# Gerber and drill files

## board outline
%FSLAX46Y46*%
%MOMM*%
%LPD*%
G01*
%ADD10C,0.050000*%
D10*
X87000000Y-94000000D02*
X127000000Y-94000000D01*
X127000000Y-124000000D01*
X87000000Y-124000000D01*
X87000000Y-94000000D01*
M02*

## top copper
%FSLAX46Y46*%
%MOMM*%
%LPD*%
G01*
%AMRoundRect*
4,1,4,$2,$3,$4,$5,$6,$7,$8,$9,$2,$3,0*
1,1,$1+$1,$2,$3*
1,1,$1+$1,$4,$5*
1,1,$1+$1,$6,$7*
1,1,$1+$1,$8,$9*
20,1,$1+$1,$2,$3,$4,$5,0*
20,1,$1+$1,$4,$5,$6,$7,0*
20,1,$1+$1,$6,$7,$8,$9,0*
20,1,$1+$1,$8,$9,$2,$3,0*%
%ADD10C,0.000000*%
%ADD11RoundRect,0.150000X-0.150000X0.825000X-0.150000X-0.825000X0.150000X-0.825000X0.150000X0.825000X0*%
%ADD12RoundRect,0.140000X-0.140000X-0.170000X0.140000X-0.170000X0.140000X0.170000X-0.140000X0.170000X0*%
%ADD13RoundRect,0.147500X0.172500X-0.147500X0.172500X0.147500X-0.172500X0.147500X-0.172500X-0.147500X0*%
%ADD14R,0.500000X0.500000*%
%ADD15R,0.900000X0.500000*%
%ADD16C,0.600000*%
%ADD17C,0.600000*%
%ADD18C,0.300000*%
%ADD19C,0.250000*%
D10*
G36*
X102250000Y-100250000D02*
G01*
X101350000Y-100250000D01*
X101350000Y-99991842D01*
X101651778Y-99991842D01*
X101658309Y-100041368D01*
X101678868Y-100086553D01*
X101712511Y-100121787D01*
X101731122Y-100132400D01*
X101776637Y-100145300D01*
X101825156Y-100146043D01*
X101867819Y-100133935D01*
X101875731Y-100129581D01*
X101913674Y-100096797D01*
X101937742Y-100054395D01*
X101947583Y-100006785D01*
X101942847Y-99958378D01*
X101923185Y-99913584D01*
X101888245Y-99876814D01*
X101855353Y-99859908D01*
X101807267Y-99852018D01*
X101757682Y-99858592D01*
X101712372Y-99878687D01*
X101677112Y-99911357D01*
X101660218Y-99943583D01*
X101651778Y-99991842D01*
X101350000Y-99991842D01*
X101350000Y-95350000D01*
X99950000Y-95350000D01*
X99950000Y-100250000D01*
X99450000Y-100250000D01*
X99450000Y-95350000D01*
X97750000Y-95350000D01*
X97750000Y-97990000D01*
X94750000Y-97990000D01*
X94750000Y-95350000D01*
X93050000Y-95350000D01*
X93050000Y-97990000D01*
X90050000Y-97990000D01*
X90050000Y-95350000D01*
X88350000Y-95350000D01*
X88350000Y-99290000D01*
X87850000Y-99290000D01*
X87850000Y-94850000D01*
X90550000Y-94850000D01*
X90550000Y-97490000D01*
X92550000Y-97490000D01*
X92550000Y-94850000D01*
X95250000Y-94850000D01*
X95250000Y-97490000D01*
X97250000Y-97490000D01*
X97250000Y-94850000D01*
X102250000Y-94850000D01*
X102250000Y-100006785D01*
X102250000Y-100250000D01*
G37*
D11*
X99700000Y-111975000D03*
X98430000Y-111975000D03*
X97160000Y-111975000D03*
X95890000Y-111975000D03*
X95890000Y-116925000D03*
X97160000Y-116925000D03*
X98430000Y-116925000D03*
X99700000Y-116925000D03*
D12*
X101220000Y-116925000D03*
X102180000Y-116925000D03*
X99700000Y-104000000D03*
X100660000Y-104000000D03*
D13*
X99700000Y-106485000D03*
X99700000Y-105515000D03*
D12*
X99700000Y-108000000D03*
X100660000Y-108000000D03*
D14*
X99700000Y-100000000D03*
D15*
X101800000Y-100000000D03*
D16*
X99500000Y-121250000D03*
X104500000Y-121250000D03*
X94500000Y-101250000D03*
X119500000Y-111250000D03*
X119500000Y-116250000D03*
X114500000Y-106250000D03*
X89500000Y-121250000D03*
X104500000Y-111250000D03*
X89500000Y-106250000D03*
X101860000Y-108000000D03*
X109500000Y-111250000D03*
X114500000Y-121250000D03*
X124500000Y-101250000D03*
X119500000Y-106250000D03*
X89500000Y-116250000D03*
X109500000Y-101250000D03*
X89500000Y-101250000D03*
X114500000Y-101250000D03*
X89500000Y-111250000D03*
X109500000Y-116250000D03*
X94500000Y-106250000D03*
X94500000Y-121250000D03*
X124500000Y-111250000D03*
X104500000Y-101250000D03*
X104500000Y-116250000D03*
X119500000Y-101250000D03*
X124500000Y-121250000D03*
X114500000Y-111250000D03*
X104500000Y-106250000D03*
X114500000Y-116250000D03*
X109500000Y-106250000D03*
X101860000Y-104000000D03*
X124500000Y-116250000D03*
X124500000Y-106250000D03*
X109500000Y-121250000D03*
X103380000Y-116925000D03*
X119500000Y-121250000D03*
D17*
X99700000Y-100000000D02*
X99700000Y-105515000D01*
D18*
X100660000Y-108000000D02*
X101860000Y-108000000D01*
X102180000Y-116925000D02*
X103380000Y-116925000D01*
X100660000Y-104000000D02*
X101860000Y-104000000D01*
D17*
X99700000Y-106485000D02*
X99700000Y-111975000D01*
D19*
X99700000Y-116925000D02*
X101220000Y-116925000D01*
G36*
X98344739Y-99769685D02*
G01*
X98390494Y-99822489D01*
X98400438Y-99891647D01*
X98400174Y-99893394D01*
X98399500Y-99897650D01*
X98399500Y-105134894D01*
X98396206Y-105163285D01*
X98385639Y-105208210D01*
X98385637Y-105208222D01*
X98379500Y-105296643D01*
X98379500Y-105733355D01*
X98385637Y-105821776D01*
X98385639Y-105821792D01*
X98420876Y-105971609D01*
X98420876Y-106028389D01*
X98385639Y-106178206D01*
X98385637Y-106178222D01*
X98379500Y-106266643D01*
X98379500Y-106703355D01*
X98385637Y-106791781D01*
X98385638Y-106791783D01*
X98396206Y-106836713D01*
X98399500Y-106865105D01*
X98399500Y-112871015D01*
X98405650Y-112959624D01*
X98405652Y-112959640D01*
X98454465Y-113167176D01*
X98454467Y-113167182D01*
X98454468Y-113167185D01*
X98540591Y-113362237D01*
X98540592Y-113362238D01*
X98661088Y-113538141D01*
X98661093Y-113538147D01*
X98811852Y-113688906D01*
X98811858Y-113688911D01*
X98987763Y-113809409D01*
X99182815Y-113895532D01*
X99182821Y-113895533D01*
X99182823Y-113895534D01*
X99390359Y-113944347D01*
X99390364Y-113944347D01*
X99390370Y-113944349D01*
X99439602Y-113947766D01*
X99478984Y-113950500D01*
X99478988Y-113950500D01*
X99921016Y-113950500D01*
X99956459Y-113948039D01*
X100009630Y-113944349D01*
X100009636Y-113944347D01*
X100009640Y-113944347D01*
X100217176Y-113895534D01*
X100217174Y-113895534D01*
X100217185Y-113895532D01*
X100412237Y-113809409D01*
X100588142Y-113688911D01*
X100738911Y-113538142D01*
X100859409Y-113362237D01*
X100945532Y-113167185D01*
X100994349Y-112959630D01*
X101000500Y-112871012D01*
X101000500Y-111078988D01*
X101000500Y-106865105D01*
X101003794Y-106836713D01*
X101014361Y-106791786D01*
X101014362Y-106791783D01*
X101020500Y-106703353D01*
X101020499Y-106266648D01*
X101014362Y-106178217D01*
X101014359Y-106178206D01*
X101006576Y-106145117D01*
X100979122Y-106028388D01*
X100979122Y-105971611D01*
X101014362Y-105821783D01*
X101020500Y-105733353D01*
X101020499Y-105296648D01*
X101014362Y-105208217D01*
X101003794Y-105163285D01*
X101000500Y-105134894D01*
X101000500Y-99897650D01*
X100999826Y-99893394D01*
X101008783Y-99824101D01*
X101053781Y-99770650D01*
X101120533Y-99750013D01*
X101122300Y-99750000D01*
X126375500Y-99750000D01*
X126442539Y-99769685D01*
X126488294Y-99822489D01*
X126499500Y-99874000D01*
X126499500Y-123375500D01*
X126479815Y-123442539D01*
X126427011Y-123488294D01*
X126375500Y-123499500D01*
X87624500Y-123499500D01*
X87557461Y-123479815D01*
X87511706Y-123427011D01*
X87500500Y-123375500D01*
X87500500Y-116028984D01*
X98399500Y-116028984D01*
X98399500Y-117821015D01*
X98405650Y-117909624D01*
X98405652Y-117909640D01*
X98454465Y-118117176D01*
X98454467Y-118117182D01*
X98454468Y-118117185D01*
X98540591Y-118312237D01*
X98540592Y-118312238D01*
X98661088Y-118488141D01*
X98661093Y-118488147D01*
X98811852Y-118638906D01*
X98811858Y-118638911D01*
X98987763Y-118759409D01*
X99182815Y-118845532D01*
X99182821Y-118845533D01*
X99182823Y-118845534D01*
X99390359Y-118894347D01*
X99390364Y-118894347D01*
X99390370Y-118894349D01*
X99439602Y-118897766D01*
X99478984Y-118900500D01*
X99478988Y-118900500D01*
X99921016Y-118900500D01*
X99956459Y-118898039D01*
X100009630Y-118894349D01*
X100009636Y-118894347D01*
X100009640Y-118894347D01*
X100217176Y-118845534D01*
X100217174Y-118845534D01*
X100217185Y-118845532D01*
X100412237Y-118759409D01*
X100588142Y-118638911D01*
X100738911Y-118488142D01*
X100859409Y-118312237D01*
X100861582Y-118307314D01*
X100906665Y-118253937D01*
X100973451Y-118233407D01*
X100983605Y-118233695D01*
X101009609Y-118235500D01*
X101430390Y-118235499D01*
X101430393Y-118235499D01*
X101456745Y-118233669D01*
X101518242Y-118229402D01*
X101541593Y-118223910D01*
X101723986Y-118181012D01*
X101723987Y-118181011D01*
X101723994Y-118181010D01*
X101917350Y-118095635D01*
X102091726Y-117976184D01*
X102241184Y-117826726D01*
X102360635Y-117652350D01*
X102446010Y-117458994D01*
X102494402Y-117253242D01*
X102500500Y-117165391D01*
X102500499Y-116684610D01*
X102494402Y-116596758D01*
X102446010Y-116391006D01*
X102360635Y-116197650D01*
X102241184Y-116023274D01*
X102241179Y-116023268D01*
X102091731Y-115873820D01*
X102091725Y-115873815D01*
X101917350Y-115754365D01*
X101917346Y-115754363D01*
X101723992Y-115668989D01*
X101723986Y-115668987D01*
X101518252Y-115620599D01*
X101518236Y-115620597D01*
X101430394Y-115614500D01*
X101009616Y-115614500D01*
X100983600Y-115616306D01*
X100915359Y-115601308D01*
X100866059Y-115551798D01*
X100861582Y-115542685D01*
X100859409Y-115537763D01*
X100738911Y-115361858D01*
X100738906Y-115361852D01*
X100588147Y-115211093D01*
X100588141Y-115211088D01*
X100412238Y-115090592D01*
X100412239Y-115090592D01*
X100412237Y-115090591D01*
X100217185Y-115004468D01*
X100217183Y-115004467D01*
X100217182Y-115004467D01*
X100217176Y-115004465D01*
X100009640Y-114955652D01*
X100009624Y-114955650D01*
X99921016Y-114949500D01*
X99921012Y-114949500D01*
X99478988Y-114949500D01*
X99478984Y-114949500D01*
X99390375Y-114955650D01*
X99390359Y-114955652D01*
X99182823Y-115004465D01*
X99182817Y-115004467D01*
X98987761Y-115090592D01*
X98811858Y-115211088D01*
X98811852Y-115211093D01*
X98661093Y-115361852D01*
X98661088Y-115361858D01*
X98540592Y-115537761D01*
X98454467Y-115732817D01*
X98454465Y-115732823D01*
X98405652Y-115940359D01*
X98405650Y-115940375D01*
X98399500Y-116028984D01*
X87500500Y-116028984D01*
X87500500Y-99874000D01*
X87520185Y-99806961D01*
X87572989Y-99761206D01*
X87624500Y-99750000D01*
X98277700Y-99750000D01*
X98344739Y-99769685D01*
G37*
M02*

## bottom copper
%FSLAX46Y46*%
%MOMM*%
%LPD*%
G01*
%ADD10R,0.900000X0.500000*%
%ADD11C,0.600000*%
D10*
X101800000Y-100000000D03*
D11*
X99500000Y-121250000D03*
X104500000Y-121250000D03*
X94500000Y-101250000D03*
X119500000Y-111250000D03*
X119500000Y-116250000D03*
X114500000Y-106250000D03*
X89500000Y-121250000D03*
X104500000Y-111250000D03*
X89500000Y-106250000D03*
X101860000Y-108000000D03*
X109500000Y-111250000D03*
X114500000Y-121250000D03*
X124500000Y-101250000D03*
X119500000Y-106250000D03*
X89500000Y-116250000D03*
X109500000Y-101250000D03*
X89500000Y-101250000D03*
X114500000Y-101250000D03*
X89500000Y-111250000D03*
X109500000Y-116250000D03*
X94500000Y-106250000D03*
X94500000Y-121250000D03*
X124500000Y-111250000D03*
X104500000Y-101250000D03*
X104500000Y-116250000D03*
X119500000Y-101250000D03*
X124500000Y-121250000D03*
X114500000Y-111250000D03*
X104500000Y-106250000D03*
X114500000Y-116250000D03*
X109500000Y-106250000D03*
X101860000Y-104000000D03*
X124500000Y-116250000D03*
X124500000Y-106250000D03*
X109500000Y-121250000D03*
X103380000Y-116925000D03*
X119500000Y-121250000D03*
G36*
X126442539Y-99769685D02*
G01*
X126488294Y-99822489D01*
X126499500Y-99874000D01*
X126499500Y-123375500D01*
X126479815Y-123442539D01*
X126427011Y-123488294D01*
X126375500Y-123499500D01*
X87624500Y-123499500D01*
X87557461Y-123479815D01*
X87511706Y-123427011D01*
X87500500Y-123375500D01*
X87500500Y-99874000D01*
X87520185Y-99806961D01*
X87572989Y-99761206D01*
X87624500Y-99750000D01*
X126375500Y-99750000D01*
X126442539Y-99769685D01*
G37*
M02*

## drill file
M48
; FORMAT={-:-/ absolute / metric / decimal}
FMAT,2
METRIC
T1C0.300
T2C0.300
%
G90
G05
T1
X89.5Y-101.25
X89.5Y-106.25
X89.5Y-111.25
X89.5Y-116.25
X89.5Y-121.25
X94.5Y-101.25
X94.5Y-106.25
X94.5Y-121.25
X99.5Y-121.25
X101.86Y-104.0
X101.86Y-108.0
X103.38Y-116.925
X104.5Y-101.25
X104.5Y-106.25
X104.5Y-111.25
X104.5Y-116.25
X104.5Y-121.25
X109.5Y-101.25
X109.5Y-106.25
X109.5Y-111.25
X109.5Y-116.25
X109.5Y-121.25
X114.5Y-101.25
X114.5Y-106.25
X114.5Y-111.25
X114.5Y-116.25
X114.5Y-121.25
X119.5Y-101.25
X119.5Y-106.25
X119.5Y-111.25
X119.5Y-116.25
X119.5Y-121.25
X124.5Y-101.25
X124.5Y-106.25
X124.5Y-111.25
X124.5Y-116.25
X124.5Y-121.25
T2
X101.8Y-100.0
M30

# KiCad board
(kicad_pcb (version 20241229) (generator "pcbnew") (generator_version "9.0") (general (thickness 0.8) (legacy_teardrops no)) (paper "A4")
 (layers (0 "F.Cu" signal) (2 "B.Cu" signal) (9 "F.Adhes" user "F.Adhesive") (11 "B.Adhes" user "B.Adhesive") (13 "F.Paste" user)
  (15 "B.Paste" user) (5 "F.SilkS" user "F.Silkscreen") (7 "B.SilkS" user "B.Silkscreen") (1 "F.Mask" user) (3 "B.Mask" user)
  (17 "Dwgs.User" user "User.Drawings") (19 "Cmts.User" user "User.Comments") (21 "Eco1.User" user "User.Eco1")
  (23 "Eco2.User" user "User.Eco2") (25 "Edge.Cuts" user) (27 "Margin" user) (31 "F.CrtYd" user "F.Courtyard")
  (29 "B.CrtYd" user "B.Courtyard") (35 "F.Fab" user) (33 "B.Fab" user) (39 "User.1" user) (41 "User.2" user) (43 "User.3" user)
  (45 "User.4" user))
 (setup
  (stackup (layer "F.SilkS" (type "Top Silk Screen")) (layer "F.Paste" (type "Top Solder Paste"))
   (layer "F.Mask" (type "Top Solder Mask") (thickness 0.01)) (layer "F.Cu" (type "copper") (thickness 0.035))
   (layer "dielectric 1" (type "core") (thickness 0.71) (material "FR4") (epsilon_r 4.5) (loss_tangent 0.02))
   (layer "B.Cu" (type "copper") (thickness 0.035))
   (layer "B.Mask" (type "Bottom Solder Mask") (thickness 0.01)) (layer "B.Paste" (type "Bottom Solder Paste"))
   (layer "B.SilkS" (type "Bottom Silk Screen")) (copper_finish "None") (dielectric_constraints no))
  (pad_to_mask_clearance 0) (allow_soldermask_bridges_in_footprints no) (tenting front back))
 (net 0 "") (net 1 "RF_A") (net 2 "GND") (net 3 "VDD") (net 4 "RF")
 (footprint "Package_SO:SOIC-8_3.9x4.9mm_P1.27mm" (layer "F.Cu") (at 97.795 114.45 -90)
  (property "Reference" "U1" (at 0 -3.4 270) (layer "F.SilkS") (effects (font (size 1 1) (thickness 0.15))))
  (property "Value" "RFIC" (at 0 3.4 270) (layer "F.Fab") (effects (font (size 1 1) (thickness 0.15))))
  (pad "1" smd roundrect (at -2.475 -1.905 270) (size 1.95 0.6) (layers "F.Cu" "F.Mask" "F.Paste") (roundrect_rratio 0.25) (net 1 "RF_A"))
  (pad "2" smd roundrect (at -2.475 -0.635 270) (size 1.95 0.6) (layers "F.Cu" "F.Mask" "F.Paste") (roundrect_rratio 0.25) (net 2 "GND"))
  (pad "3" smd roundrect (at -2.475 0.635 270) (size 1.95 0.6) (layers "F.Cu" "F.Mask" "F.Paste") (roundrect_rratio 0.25) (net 2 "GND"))
  (pad "4" smd roundrect (at -2.475 1.905 270) (size 1.95 0.6) (layers "F.Cu" "F.Mask" "F.Paste") (roundrect_rratio 0.25) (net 2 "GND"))
  (pad "5" smd roundrect (at 2.475 1.905 270) (size 1.95 0.6) (layers "F.Cu" "F.Mask" "F.Paste") (roundrect_rratio 0.25) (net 2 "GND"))
  (pad "6" smd roundrect (at 2.475 0.635 270) (size 1.95 0.6) (layers "F.Cu" "F.Mask" "F.Paste") (roundrect_rratio 0.25) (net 2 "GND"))
  (pad "7" smd roundrect (at 2.475 -0.635 270) (size 1.95 0.6) (layers "F.Cu" "F.Mask" "F.Paste") (roundrect_rratio 0.25) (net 2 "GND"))
  (pad "8" smd roundrect (at 2.475 -1.905 270) (size 1.95 0.6) (layers "F.Cu" "F.Mask" "F.Paste") (roundrect_rratio 0.25) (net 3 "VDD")))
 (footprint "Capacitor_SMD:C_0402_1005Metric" (layer "F.Cu") (at 101.7 116.925)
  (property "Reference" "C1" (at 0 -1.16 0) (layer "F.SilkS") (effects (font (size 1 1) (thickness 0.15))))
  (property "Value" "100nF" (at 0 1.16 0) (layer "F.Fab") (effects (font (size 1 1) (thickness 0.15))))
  (pad "1" smd roundrect (at -0.48 0) (size 0.56 0.62) (layers "F.Cu" "F.Mask" "F.Paste") (roundrect_rratio 0.25) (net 3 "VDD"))
  (pad "2" smd roundrect (at 0.48 0) (size 0.56 0.62) (layers "F.Cu" "F.Mask" "F.Paste") (roundrect_rratio 0.25) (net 2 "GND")))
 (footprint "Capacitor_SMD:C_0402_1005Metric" (layer "F.Cu") (at 100.18 104)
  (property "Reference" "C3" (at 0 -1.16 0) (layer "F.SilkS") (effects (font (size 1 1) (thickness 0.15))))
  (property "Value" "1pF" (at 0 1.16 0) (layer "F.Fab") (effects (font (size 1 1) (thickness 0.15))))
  (pad "1" smd roundrect (at -0.48 0) (size 0.56 0.62) (layers "F.Cu" "F.Mask" "F.Paste") (roundrect_rratio 0.25) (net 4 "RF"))
  (pad "2" smd roundrect (at 0.48 0) (size 0.56 0.62) (layers "F.Cu" "F.Mask" "F.Paste") (roundrect_rratio 0.25) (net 2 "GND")))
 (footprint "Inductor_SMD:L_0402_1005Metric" (layer "F.Cu") (at 99.7 106 90)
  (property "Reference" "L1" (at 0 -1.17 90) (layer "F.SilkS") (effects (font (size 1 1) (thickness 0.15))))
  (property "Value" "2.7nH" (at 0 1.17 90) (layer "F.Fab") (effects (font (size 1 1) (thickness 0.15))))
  (pad "1" smd roundrect (at -0.485 0 90) (size 0.59 0.64) (layers "F.Cu" "F.Mask" "F.Paste") (roundrect_rratio 0.25) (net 1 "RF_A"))
  (pad "2" smd roundrect (at 0.485 0 90) (size 0.59 0.64) (layers "F.Cu" "F.Mask" "F.Paste") (roundrect_rratio 0.25) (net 4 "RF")))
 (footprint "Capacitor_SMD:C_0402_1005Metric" (layer "F.Cu") (at 100.18 108)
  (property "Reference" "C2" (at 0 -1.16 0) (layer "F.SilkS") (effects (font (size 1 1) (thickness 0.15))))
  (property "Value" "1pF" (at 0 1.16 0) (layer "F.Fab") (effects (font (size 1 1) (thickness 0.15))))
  (pad "1" smd roundrect (at -0.48 0) (size 0.56 0.62) (layers "F.Cu" "F.Mask" "F.Paste") (roundrect_rratio 0.25) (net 1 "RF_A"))
  (pad "2" smd roundrect (at 0.48 0) (size 0.56 0.62) (layers "F.Cu" "F.Mask" "F.Paste") (roundrect_rratio 0.25) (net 2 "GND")))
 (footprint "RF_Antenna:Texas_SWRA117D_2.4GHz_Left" (layer "F.Cu") (at 99.7 100)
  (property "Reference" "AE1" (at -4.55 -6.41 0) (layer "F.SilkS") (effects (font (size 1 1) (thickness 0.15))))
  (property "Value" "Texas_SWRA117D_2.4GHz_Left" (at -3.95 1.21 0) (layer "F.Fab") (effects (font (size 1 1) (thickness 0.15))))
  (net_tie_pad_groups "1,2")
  (fp_poly
   (pts (xy -2.45 -2.51) (xy -4.45 -2.51) (xy -4.45 -5.15) (xy -7.15 -5.15) (xy -7.15 -2.51) (xy -9.15 -2.51) (xy -9.15 -5.15)
    (xy -11.85 -5.15) (xy -11.85 -0.71) (xy -11.35 -0.71) (xy -11.35 -4.65) (xy -9.65 -4.65) (xy -9.65 -2.01) (xy -6.65 -2.01)
    (xy -6.65 -4.65) (xy -4.95 -4.65) (xy -4.95 -2.01) (xy -1.95 -2.01) (xy -1.95 -4.65) (xy -0.25 -4.65) (xy -0.25 0.25) (xy 0.25 0.25)
    (xy 0.25 -4.65) (xy 1.65 -4.65) (xy 1.65 0.25) (xy 2.55 0.25) (xy 2.55 0.006785) (xy 2.247583 0.006785) (xy 2.237742 0.054395)
    (xy 2.213674 0.096797) (xy 2.175731 0.129581) (xy 2.167819 0.133935) (xy 2.125156 0.146043) (xy 2.076637 0.1453) (xy 2.031122 0.1324)
    (xy 2.012511 0.121787) (xy 1.978868 0.086553) (xy 1.958309 0.041368) (xy 1.951778 -0.008158) (xy 1.960218 -0.056417)
    (xy 1.977112 -0.088643) (xy 2.012372 -0.121313) (xy 2.057682 -0.141408) (xy 2.107267 -0.147982) (xy 2.155353 -0.140092)
    (xy 2.188245 -0.123186) (xy 2.223185 -0.086416) (xy 2.242847 -0.041622) (xy 2.247583 0.006785) (xy 2.55 0.006785) (xy 2.55 -5.15)
    (xy -2.45 -5.15) (xy -2.45 -2.51))
   (stroke (width 0) (type solid)) (fill yes) (layer "F.Cu"))
  (pad "1" connect rect (at 0 0) (size 0.5 0.5) (layers "F.Cu") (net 4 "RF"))
  (pad "2" thru_hole rect (at 2.1 0) (size 0.9 0.5) (drill 0.3) (layers "*.Cu") (remove_unused_layers no) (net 2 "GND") (zone_connect 2)))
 (gr_rect (start 87 94) (end 127 124) (stroke (width 0.05) (type default)) (fill no) (layer "Edge.Cuts"))
 (segment (start 99.7 100) (end 99.7 105.515) (width 0.6) (layer "F.Cu") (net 4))
 (segment (start 100.66 108) (end 101.86 108) (width 0.3) (layer "F.Cu") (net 2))
 (segment (start 102.18 116.925) (end 103.38 116.925) (width 0.3) (layer "F.Cu") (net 2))
 (segment (start 100.66 104) (end 101.86 104) (width 0.3) (layer "F.Cu") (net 2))
 (via (at 99.5 121.25) (size 0.6) (drill 0.3) (layers "F.Cu" "B.Cu") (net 2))
 (via (at 104.5 121.25) (size 0.6) (drill 0.3) (layers "F.Cu" "B.Cu") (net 2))
 (via (at 94.5 101.25) (size 0.6) (drill 0.3) (layers "F.Cu" "B.Cu") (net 2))
 (via (at 119.5 111.25) (size 0.6) (drill 0.3) (layers "F.Cu" "B.Cu") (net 2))
 (via (at 119.5 116.25) (size 0.6) (drill 0.3) (layers "F.Cu" "B.Cu") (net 2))
 (via (at 114.5 106.25) (size 0.6) (drill 0.3) (layers "F.Cu" "B.Cu") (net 2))
 (via (at 89.5 121.25) (size 0.6) (drill 0.3) (layers "F.Cu" "B.Cu") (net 2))
 (via (at 104.5 111.25) (size 0.6) (drill 0.3) (layers "F.Cu" "B.Cu") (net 2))
 (via (at 89.5 106.25) (size 0.6) (drill 0.3) (layers "F.Cu" "B.Cu") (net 2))
 (via (at 101.86 108) (size 0.6) (drill 0.3) (layers "F.Cu" "B.Cu") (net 2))
 (via (at 109.5 111.25) (size 0.6) (drill 0.3) (layers "F.Cu" "B.Cu") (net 2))
 (via (at 114.5 121.25) (size 0.6) (drill 0.3) (layers "F.Cu" "B.Cu") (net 2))
 (via (at 124.5 101.25) (size 0.6) (drill 0.3) (layers "F.Cu" "B.Cu") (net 2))
 (via (at 119.5 106.25) (size 0.6) (drill 0.3) (layers "F.Cu" "B.Cu") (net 2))
 (via (at 89.5 116.25) (size 0.6) (drill 0.3) (layers "F.Cu" "B.Cu") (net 2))
 (via (at 109.5 101.25) (size 0.6) (drill 0.3) (layers "F.Cu" "B.Cu") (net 2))
 (via (at 89.5 101.25) (size 0.6) (drill 0.3) (layers "F.Cu" "B.Cu") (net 2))
 (via (at 114.5 101.25) (size 0.6) (drill 0.3) (layers "F.Cu" "B.Cu") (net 2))
 (via (at 89.5 111.25) (size 0.6) (drill 0.3) (layers "F.Cu" "B.Cu") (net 2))
 (via (at 109.5 116.25) (size 0.6) (drill 0.3) (layers "F.Cu" "B.Cu") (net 2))
 (via (at 94.5 106.25) (size 0.6) (drill 0.3) (layers "F.Cu" "B.Cu") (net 2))
 (via (at 94.5 121.25) (size 0.6) (drill 0.3) (layers "F.Cu" "B.Cu") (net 2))
 (via (at 124.5 111.25) (size 0.6) (drill 0.3) (layers "F.Cu" "B.Cu") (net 2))
 (via (at 104.5 101.25) (size 0.6) (drill 0.3) (layers "F.Cu" "B.Cu") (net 2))
 (via (at 104.5 116.25) (size 0.6) (drill 0.3) (layers "F.Cu" "B.Cu") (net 2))
 (via (at 119.5 101.25) (size 0.6) (drill 0.3) (layers "F.Cu" "B.Cu") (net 2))
 (via (at 124.5 121.25) (size 0.6) (drill 0.3) (layers "F.Cu" "B.Cu") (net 2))
 (via (at 114.5 111.25) (size 0.6) (drill 0.3) (layers "F.Cu" "B.Cu") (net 2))
 (via (at 104.5 106.25) (size 0.6) (drill 0.3) (layers "F.Cu" "B.Cu") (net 2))
 (via (at 114.5 116.25) (size 0.6) (drill 0.3) (layers "F.Cu" "B.Cu") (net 2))
 (via (at 109.5 106.25) (size 0.6) (drill 0.3) (layers "F.Cu" "B.Cu") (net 2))
 (via (at 101.86 104) (size 0.6) (drill 0.3) (layers "F.Cu" "B.Cu") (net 2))
 (via (at 124.5 116.25) (size 0.6) (drill 0.3) (layers "F.Cu" "B.Cu") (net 2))
 (via (at 124.5 106.25) (size 0.6) (drill 0.3) (layers "F.Cu" "B.Cu") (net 2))
 (via (at 109.5 121.25) (size 0.6) (drill 0.3) (layers "F.Cu" "B.Cu") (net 2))
 (via (at 103.38 116.925) (size 0.6) (drill 0.3) (layers "F.Cu" "B.Cu") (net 2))
 (via (at 119.5 121.25) (size 0.6) (drill 0.3) (layers "F.Cu" "B.Cu") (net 2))
 (segment (start 99.7 106.485) (end 99.7 111.975) (width 0.6) (layer "F.Cu") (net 1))
 (segment (start 99.7 116.925) (end 101.22 116.925) (width 0.25) (layer "F.Cu") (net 3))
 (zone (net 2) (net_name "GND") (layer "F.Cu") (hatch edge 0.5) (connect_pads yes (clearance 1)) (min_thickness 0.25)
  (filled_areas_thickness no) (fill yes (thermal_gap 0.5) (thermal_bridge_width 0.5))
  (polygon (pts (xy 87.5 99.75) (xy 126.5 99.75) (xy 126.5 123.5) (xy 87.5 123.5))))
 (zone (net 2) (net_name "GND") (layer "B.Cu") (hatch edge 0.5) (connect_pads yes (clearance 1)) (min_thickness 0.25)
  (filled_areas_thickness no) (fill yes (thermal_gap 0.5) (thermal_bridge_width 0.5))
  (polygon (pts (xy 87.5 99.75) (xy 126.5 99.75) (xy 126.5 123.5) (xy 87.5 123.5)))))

